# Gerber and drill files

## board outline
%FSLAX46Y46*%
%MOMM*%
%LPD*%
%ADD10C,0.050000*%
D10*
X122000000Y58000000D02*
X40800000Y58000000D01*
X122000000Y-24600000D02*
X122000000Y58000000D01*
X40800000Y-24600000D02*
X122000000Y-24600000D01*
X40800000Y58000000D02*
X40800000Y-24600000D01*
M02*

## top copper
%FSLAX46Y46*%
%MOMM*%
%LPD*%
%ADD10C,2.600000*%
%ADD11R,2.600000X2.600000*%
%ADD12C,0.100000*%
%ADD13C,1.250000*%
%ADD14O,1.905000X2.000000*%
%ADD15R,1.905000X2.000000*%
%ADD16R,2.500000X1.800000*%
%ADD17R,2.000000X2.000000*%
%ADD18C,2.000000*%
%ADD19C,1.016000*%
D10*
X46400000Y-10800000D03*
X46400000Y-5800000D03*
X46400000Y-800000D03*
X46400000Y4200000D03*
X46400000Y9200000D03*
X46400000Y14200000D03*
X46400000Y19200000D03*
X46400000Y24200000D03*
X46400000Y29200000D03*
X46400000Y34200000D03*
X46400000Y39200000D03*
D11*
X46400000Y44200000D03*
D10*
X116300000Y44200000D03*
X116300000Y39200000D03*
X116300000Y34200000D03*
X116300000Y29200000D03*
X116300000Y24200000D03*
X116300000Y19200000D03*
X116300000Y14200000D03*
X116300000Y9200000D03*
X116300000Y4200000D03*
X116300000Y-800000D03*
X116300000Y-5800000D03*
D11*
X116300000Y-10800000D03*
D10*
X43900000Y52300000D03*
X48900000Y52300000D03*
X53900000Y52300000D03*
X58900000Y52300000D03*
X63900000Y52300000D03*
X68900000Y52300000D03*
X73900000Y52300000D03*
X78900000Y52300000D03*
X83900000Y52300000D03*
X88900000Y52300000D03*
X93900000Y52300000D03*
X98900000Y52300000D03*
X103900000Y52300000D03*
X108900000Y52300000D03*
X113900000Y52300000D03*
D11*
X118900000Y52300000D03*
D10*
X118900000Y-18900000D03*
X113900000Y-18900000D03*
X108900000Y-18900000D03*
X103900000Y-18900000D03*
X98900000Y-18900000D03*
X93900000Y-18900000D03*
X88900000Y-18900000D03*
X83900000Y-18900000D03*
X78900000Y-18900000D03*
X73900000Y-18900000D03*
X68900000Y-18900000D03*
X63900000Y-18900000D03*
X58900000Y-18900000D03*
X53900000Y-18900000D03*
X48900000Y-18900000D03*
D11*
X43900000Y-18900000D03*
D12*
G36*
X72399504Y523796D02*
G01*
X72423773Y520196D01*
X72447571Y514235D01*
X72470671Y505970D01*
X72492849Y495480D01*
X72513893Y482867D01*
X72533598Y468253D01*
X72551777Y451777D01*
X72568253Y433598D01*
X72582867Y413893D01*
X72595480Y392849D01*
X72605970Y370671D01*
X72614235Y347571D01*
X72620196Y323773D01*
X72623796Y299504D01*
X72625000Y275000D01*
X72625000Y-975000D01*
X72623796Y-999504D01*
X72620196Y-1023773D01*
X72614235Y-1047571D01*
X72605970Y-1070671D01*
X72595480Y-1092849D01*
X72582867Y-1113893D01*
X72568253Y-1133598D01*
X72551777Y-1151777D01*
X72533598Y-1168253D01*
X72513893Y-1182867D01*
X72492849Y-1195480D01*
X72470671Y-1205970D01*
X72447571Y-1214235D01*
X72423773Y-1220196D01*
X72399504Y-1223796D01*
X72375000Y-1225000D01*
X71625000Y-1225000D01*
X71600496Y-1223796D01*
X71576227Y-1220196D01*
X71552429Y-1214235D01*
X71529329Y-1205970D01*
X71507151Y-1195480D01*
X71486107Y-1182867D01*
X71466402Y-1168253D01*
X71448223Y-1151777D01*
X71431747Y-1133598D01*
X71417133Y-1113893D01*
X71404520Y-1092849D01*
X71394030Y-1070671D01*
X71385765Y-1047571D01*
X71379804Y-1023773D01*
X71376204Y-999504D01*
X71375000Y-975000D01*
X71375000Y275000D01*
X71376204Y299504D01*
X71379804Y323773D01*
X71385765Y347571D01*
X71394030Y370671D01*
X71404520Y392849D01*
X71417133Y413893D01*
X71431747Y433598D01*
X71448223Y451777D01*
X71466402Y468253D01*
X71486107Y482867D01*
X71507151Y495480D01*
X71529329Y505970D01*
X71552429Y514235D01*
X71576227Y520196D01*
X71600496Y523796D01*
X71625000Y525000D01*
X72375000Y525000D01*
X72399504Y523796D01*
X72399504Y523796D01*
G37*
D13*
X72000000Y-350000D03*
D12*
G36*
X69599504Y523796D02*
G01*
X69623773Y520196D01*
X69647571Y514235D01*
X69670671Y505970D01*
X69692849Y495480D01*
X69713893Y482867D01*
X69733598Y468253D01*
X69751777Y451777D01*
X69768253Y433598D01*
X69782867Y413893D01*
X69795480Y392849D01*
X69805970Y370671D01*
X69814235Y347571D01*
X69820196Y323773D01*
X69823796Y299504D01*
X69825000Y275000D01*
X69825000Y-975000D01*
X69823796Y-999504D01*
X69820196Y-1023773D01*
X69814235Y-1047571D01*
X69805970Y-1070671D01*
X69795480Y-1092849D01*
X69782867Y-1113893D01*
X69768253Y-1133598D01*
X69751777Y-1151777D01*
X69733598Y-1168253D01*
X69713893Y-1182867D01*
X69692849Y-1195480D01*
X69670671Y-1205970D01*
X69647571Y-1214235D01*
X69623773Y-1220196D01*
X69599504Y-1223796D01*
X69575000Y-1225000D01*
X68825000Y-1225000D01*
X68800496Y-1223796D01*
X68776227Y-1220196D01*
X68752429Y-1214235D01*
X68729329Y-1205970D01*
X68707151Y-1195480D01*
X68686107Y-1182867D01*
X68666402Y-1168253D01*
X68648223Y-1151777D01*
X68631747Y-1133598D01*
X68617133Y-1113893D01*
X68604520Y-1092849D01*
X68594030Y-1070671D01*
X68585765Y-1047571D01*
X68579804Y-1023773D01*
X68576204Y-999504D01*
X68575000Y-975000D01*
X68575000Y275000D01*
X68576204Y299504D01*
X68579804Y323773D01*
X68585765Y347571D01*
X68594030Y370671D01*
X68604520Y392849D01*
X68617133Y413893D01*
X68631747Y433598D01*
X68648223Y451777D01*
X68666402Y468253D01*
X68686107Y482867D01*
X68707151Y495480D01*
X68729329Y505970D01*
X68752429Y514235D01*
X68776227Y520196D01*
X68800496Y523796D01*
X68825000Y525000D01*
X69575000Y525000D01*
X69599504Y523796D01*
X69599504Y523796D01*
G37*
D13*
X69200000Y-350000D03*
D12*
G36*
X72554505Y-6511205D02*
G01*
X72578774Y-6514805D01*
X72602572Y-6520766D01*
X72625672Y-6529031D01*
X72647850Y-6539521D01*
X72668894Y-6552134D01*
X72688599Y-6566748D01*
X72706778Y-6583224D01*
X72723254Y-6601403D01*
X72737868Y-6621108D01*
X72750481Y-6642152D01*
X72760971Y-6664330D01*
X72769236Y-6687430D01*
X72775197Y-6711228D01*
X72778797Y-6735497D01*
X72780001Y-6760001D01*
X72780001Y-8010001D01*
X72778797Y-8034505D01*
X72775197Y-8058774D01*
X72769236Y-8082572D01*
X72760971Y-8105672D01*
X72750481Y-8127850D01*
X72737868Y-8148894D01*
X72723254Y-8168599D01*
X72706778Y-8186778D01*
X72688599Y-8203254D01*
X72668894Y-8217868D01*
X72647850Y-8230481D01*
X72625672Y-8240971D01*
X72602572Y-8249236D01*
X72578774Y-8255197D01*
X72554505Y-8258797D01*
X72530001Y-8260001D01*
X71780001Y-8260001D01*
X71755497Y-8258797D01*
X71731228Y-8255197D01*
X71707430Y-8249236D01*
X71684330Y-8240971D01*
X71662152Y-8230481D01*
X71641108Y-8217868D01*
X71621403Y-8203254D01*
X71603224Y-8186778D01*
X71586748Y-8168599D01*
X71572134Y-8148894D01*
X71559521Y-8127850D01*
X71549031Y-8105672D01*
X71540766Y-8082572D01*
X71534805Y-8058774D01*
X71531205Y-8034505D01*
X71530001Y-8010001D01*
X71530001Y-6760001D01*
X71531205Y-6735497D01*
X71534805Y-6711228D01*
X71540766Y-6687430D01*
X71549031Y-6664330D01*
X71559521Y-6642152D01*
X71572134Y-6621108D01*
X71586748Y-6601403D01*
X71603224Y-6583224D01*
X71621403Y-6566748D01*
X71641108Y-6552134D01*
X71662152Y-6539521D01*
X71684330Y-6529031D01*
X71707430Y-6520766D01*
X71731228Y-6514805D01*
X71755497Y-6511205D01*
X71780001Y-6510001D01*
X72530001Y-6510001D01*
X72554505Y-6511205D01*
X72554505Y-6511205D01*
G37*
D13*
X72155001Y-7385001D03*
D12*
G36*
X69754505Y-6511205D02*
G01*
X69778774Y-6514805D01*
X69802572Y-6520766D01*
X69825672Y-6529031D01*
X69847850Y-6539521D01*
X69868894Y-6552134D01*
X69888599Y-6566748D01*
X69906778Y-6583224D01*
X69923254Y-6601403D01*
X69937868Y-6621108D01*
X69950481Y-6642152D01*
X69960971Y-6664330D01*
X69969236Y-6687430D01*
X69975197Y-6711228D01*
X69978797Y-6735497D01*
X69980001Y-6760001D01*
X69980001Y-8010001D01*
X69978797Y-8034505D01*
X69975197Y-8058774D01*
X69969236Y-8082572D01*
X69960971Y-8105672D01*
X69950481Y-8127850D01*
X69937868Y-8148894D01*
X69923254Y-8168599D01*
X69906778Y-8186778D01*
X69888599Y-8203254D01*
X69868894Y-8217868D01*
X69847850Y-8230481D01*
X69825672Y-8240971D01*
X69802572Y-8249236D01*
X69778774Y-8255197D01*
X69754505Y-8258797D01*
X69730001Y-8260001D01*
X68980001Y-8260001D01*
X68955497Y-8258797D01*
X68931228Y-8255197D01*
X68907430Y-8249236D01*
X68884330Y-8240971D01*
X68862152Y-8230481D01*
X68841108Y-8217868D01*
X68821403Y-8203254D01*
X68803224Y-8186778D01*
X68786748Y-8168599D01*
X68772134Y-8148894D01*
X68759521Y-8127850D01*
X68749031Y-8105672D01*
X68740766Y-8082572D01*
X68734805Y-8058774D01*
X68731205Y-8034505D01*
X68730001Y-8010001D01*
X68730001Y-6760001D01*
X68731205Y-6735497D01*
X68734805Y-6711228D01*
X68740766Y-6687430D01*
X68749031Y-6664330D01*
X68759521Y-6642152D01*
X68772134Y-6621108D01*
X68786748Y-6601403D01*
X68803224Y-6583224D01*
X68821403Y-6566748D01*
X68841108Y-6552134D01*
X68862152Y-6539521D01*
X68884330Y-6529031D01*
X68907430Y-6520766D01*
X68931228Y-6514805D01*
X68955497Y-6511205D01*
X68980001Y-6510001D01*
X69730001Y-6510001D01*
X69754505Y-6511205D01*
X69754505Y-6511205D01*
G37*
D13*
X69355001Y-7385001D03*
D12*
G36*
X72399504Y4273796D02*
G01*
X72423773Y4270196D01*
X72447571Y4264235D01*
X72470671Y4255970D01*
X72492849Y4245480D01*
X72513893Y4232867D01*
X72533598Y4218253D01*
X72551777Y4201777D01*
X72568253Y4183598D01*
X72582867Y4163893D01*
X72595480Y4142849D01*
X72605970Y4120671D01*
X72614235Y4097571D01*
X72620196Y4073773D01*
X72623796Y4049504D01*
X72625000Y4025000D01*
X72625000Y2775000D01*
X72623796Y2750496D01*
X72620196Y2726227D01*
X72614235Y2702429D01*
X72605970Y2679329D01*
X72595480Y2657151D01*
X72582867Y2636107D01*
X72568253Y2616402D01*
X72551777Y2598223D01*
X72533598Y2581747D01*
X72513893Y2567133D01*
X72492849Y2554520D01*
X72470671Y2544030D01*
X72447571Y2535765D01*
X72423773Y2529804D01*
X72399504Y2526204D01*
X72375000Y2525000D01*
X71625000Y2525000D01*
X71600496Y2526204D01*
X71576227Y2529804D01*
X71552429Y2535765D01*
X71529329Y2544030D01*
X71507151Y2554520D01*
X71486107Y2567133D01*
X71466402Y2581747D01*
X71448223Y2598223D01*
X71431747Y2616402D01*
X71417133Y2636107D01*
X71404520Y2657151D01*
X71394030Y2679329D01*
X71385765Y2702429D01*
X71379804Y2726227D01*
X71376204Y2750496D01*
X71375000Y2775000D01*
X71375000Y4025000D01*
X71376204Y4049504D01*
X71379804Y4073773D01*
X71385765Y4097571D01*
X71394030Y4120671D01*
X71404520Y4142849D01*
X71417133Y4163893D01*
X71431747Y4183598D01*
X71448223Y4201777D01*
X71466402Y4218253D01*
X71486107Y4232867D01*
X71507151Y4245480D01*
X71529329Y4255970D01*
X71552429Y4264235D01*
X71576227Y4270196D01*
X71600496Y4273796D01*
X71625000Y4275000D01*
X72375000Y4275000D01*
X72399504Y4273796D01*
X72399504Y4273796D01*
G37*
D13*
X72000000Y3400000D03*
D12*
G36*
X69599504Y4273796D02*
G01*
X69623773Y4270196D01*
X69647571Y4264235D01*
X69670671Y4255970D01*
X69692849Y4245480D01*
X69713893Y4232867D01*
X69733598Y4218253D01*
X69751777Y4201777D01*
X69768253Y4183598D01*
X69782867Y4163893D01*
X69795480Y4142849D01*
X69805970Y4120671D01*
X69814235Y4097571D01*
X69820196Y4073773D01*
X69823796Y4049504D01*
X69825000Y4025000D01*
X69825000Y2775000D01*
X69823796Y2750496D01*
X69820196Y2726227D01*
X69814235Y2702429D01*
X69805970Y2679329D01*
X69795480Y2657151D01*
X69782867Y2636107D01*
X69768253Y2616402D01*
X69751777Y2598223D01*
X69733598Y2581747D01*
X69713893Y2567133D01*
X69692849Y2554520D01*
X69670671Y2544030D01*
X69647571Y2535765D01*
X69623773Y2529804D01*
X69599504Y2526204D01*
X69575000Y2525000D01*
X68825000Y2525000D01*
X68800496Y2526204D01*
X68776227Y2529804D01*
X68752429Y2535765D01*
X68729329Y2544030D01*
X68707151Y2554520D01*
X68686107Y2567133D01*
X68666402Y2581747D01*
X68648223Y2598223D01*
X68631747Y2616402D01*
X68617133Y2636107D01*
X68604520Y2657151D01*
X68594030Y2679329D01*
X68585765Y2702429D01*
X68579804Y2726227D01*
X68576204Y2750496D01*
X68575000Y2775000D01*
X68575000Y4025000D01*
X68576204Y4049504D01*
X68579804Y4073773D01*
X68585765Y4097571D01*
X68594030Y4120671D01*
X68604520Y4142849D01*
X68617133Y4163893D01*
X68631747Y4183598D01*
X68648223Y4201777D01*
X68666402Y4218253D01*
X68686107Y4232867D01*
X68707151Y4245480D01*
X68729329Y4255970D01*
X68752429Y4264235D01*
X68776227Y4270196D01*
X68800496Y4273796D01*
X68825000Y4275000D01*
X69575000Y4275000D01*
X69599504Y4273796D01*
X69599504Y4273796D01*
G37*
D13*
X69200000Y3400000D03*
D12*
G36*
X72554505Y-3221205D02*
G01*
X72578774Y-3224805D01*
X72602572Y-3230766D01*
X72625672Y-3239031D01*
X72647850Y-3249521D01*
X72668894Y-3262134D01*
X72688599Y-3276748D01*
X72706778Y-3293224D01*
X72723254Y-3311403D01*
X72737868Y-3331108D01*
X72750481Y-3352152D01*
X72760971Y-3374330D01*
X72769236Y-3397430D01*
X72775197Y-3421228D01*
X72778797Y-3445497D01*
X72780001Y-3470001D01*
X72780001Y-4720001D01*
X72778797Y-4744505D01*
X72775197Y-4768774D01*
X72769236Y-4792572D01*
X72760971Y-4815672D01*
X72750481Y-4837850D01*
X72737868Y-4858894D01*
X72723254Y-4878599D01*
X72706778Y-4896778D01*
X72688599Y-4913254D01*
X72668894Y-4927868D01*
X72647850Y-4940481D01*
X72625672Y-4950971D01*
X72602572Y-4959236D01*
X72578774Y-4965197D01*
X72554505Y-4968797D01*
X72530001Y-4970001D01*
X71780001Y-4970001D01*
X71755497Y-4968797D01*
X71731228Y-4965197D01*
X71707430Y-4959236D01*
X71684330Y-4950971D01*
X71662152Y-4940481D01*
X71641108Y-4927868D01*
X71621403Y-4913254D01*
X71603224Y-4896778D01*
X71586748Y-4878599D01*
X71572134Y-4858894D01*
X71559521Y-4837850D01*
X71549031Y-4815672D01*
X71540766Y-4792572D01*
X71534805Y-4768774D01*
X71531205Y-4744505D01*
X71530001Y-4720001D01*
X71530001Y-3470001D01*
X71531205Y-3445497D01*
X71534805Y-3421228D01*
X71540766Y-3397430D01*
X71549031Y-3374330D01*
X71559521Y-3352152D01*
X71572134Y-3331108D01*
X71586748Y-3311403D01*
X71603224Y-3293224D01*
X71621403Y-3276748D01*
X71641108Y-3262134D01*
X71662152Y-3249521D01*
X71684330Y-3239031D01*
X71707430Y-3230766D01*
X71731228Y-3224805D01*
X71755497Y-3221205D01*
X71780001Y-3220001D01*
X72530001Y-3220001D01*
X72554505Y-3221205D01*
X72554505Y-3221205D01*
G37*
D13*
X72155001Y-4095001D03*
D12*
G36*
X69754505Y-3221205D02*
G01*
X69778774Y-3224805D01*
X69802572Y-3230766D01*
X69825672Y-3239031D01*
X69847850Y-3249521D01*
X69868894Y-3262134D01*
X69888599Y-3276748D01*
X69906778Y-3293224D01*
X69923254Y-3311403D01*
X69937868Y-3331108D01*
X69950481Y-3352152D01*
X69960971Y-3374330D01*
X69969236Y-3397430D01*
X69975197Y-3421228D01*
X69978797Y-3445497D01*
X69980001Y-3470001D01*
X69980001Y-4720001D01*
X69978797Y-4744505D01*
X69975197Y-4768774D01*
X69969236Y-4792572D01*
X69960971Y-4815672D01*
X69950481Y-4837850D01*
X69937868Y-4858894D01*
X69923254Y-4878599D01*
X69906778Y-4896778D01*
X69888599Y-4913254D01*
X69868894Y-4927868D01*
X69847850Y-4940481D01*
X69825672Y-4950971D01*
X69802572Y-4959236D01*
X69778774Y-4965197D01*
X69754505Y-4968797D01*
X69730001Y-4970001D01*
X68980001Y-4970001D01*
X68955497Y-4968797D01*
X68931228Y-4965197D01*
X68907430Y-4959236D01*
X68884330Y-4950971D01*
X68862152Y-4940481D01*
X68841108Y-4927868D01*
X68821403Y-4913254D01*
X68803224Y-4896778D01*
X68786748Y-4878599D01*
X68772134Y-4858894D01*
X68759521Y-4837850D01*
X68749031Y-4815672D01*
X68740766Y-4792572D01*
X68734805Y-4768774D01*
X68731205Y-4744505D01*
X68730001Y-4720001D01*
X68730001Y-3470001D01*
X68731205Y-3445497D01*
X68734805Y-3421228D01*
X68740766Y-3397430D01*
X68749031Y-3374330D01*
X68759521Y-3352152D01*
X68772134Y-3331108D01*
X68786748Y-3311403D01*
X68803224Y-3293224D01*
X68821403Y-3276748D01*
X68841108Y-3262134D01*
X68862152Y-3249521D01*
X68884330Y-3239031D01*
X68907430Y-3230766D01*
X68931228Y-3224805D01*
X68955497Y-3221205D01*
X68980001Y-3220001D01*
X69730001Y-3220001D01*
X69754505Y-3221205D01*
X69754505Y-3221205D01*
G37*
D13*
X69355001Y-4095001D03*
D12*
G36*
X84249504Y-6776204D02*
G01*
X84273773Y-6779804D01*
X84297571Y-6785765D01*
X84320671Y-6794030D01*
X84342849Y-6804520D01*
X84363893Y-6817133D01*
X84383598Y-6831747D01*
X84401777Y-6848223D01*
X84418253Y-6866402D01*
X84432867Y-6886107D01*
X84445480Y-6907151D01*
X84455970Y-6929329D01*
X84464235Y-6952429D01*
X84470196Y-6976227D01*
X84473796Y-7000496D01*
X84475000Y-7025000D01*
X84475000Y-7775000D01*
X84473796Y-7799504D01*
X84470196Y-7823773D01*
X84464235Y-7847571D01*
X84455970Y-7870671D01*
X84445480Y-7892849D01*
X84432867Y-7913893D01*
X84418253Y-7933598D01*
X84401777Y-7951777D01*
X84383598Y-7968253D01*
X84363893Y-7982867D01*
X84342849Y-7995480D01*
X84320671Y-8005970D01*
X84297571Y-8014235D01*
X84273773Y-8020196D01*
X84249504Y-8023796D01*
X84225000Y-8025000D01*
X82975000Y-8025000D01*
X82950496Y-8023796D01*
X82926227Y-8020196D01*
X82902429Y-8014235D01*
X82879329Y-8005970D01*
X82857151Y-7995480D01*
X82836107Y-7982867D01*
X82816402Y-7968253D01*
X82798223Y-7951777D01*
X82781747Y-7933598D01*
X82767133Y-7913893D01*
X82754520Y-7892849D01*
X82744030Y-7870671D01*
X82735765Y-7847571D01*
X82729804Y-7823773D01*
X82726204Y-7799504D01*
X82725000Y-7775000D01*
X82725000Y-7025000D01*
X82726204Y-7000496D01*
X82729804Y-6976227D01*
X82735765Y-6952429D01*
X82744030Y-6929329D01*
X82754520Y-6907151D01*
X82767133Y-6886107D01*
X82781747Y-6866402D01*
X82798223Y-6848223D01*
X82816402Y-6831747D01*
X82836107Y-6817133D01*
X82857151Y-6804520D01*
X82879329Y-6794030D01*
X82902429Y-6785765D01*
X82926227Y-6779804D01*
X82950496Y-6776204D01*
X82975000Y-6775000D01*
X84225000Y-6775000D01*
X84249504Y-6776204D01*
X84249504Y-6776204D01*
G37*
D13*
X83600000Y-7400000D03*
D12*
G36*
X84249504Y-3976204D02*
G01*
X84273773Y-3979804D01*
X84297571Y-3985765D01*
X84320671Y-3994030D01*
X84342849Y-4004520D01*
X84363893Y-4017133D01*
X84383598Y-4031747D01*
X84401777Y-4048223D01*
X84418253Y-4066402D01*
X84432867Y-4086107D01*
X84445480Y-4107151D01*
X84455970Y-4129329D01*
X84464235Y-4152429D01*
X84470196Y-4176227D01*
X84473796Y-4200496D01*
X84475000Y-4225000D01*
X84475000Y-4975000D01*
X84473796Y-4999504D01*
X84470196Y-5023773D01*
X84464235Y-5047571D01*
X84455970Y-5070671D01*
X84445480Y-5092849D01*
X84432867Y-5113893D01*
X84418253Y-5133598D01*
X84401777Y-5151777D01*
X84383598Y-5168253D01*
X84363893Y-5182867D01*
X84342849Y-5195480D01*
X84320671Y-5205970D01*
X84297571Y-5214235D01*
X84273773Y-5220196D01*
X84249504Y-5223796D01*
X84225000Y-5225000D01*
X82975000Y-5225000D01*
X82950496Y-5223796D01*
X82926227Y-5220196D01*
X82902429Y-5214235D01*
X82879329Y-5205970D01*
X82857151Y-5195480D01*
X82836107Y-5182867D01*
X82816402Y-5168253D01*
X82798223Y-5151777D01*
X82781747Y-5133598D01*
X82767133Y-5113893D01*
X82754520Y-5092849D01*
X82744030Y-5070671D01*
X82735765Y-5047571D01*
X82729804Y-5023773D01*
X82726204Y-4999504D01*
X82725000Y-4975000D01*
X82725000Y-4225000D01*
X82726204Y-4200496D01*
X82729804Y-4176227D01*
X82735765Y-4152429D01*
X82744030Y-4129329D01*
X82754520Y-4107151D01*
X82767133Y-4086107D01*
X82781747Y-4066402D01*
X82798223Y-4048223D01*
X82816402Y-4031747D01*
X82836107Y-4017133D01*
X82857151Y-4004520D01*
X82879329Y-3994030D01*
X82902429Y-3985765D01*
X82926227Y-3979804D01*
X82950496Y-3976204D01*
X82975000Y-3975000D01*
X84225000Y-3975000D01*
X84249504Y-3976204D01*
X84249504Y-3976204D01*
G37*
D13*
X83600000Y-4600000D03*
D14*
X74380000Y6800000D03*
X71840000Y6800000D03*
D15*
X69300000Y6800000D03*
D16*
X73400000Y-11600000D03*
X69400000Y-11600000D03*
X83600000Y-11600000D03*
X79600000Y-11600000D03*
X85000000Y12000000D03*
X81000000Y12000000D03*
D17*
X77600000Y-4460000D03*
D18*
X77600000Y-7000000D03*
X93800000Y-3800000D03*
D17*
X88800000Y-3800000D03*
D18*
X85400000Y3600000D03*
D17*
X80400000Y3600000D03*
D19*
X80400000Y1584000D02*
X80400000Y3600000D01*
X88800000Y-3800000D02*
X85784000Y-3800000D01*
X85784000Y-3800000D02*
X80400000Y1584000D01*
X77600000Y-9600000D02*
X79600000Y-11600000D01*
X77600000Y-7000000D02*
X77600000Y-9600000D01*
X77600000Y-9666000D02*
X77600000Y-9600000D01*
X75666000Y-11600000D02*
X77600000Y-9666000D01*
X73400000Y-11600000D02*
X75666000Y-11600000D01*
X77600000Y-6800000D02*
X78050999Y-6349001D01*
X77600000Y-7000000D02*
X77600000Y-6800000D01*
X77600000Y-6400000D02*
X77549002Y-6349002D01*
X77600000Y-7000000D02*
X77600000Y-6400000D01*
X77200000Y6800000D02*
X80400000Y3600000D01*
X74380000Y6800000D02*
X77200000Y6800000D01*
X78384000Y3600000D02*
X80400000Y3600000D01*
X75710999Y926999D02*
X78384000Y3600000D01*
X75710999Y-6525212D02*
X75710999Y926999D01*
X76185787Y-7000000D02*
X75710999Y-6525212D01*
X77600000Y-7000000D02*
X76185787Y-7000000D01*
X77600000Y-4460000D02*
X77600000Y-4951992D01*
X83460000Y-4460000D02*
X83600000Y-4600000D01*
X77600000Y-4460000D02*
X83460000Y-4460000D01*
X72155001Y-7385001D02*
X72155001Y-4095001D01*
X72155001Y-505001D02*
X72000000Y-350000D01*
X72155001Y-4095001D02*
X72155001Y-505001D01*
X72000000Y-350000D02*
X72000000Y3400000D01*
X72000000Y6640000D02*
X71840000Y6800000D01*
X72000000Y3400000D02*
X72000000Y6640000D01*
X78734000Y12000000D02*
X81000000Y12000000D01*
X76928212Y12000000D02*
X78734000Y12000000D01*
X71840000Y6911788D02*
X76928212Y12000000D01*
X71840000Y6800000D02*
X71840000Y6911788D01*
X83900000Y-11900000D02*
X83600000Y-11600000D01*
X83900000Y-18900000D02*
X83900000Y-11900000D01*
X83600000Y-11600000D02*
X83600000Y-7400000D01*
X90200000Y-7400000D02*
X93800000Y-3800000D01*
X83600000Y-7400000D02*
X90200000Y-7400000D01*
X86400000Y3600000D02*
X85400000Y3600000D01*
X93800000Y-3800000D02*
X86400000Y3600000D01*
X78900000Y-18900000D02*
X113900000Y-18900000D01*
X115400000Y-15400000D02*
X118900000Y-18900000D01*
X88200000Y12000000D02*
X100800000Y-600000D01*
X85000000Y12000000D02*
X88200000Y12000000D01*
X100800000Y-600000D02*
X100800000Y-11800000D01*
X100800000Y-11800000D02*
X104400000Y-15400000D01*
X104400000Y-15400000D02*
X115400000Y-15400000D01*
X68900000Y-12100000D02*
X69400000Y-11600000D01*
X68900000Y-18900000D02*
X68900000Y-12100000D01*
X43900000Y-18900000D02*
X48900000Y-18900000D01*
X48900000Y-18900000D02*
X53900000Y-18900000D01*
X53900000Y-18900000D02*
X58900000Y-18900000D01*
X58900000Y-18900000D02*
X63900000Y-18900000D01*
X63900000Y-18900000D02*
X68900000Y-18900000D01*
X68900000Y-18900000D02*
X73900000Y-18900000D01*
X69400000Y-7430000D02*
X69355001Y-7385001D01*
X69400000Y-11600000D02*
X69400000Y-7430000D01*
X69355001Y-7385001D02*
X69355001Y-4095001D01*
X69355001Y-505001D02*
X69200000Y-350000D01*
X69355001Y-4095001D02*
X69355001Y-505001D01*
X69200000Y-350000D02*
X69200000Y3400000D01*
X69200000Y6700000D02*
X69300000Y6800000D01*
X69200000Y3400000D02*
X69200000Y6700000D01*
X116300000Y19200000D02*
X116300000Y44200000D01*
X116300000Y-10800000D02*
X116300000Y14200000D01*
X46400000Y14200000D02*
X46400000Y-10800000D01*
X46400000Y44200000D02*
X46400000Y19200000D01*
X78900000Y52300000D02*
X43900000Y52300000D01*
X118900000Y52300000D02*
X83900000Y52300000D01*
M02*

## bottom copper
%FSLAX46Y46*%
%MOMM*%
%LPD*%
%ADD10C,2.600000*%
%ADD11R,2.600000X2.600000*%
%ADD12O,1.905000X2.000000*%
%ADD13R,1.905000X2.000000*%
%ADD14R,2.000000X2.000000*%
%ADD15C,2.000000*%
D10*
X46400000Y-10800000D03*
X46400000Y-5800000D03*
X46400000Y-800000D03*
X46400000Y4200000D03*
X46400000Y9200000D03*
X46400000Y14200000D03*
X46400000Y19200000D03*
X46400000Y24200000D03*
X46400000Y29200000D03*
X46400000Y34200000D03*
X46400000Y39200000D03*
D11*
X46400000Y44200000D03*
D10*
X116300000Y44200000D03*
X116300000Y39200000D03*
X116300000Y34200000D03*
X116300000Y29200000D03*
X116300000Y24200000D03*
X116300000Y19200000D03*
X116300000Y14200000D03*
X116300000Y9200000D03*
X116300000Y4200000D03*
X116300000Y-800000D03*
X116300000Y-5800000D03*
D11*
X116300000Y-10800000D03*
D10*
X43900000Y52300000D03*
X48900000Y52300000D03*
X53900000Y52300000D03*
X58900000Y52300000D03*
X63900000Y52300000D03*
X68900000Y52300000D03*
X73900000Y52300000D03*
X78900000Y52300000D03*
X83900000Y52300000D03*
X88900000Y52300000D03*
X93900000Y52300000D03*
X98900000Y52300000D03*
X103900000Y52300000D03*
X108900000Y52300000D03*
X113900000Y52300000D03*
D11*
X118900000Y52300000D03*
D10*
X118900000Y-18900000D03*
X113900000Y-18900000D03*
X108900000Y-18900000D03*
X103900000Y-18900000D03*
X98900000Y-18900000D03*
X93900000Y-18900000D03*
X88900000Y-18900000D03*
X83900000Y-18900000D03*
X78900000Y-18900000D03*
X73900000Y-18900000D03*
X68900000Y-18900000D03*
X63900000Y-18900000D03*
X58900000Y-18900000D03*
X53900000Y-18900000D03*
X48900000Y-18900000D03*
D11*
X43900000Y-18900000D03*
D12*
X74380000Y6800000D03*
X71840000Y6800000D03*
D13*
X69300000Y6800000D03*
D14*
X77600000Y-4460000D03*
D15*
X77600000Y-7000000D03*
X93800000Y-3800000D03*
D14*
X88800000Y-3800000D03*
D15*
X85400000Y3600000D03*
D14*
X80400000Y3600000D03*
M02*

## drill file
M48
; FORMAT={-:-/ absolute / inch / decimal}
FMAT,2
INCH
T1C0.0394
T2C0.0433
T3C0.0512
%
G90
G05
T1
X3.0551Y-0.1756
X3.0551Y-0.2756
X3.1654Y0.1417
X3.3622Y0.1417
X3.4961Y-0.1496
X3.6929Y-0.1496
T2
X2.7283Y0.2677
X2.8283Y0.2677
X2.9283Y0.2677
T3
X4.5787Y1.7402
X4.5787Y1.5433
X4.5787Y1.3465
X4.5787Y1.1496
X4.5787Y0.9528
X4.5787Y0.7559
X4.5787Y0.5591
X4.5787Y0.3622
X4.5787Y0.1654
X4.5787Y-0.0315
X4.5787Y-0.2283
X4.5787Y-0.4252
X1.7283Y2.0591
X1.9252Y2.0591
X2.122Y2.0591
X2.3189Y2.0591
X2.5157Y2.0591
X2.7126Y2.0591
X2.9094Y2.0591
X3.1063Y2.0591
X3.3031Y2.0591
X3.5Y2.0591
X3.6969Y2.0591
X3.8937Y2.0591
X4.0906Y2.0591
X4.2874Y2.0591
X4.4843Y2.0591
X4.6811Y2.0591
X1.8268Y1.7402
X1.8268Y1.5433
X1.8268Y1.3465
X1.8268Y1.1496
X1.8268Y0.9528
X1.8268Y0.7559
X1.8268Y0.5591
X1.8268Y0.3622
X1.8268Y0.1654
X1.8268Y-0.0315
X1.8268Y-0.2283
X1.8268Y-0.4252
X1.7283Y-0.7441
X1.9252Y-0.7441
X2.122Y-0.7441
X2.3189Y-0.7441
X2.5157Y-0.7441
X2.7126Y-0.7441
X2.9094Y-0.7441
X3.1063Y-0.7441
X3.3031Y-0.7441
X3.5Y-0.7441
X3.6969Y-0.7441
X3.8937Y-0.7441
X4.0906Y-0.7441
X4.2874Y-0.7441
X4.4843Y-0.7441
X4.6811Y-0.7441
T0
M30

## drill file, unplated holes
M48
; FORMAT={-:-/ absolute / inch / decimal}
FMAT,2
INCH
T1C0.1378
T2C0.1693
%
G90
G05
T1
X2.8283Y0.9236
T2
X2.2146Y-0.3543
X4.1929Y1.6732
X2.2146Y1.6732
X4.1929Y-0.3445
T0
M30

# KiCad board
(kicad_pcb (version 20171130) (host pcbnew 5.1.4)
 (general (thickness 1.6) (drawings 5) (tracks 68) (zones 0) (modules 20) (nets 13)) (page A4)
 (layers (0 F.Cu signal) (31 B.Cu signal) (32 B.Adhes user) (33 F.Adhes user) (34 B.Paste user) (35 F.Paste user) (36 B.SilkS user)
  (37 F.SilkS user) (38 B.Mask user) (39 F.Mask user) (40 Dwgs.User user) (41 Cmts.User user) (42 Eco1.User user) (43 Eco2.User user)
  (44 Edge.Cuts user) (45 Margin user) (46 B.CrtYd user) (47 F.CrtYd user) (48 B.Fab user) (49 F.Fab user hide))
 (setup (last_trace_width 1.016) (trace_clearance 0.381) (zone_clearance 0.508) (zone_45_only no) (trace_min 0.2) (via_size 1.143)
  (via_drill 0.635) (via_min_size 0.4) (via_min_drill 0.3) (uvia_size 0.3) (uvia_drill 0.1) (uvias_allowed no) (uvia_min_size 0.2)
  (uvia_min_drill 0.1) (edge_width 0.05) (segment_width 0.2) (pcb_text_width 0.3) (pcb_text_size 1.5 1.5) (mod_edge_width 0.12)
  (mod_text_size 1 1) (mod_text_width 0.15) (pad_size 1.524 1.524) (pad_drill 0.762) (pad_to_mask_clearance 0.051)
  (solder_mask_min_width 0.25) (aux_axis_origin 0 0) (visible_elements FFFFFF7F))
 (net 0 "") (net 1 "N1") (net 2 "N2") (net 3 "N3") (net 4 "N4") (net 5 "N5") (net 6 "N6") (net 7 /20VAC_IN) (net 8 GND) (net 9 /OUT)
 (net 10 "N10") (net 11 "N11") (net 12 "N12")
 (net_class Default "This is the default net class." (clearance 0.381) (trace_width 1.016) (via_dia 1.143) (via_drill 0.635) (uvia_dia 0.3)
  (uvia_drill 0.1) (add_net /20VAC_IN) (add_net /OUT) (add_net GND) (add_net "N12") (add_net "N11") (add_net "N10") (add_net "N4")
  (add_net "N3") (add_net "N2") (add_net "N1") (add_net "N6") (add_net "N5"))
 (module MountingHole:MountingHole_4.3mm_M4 (layer F.Cu) (at 56.25 -42.5)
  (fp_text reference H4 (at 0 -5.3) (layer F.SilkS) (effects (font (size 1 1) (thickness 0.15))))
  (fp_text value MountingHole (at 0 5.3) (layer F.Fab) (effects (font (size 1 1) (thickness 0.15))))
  (pad 1 np_thru_hole circle (at 0 0) (size 4.3 4.3) (drill 4.3) (layers *.Cu *.Mask)))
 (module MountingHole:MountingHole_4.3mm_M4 (layer F.Cu) (at 106.5 -42.5)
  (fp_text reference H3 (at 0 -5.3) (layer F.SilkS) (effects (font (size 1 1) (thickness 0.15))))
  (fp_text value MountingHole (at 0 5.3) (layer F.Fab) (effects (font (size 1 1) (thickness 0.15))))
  (pad 1 np_thru_hole circle (at 0 0) (size 4.3 4.3) (drill 4.3) (layers *.Cu *.Mask)))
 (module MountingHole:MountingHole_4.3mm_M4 (layer F.Cu) (at 56.25 9)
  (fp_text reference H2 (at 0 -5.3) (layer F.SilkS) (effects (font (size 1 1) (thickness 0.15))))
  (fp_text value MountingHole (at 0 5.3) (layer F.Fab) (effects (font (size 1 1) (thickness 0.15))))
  (pad 1 np_thru_hole circle (at 0 0) (size 4.3 4.3) (drill 4.3) (layers *.Cu *.Mask)))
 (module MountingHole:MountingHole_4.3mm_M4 (layer F.Cu) (at 106.5 8.75)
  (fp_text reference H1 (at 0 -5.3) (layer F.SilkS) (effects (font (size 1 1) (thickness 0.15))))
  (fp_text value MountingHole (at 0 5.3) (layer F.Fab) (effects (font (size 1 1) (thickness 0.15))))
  (pad 1 np_thru_hole circle (at 0 0) (size 4.3 4.3) (drill 4.3) (layers *.Cu *.Mask)))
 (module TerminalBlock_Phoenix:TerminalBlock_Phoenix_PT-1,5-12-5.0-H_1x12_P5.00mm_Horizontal (layer F.Cu) (at 46.4 -44.2 270)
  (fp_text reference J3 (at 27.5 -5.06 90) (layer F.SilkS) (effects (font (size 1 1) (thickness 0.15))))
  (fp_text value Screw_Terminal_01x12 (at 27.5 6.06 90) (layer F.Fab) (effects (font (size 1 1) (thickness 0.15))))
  (pad 12 thru_hole circle (at 55 0 270) (size 2.6 2.6) (drill 1.3) (layers *.Cu *.Mask) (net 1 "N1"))
  (pad 11 thru_hole circle (at 50 0 270) (size 2.6 2.6) (drill 1.3) (layers *.Cu *.Mask) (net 1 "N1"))
  (pad 10 thru_hole circle (at 45 0 270) (size 2.6 2.6) (drill 1.3) (layers *.Cu *.Mask) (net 1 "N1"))
  (pad 9 thru_hole circle (at 40 0 270) (size 2.6 2.6) (drill 1.3) (layers *.Cu *.Mask) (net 1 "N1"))
  (pad 8 thru_hole circle (at 35 0 270) (size 2.6 2.6) (drill 1.3) (layers *.Cu *.Mask) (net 1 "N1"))
  (pad 7 thru_hole circle (at 30 0 270) (size 2.6 2.6) (drill 1.3) (layers *.Cu *.Mask) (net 1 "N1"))
  (pad 6 thru_hole circle (at 25 0 270) (size 2.6 2.6) (drill 1.3) (layers *.Cu *.Mask) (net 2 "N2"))
  (pad 5 thru_hole circle (at 20 0 270) (size 2.6 2.6) (drill 1.3) (layers *.Cu *.Mask) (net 2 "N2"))
  (pad 4 thru_hole circle (at 15 0 270) (size 2.6 2.6) (drill 1.3) (layers *.Cu *.Mask) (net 2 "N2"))
  (pad 3 thru_hole circle (at 10 0 270) (size 2.6 2.6) (drill 1.3) (layers *.Cu *.Mask) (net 2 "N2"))
  (pad 2 thru_hole circle (at 5 0 270) (size 2.6 2.6) (drill 1.3) (layers *.Cu *.Mask) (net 2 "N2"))
  (pad 1 thru_hole rect (at 0 0 270) (size 2.6 2.6) (drill 1.3) (layers *.Cu *.Mask) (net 2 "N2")))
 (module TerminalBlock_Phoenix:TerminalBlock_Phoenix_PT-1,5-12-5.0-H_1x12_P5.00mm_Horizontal (layer F.Cu) (at 116.3 10.8 90)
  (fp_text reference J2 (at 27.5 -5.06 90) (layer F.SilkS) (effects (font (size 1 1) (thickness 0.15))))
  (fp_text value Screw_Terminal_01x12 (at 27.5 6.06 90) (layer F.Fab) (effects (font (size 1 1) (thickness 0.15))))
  (pad 12 thru_hole circle (at 55 0 90) (size 2.6 2.6) (drill 1.3) (layers *.Cu *.Mask) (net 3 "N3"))
  (pad 11 thru_hole circle (at 50 0 90) (size 2.6 2.6) (drill 1.3) (layers *.Cu *.Mask) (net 3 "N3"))
  (pad 10 thru_hole circle (at 45 0 90) (size 2.6 2.6) (drill 1.3) (layers *.Cu *.Mask) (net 3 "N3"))
  (pad 9 thru_hole circle (at 40 0 90) (size 2.6 2.6) (drill 1.3) (layers *.Cu *.Mask) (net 3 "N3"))
  (pad 8 thru_hole circle (at 35 0 90) (size 2.6 2.6) (drill 1.3) (layers *.Cu *.Mask) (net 3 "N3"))
  (pad 7 thru_hole circle (at 30 0 90) (size 2.6 2.6) (drill 1.3) (layers *.Cu *.Mask) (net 3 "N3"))
  (pad 6 thru_hole circle (at 25 0 90) (size 2.6 2.6) (drill 1.3) (layers *.Cu *.Mask) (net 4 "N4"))
  (pad 5 thru_hole circle (at 20 0 90) (size 2.6 2.6) (drill 1.3) (layers *.Cu *.Mask) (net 4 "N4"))
  (pad 4 thru_hole circle (at 15 0 90) (size 2.6 2.6) (drill 1.3) (layers *.Cu *.Mask) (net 4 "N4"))
  (pad 3 thru_hole circle (at 10 0 90) (size 2.6 2.6) (drill 1.3) (layers *.Cu *.Mask) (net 4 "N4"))
  (pad 2 thru_hole circle (at 5 0 90) (size 2.6 2.6) (drill 1.3) (layers *.Cu *.Mask) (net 4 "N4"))
  (pad 1 thru_hole rect (at 0 0 90) (size 2.6 2.6) (drill 1.3) (layers *.Cu *.Mask) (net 4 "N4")))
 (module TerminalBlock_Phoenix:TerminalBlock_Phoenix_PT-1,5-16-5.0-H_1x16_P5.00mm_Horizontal (layer F.Cu) (at 118.9 -52.3 180)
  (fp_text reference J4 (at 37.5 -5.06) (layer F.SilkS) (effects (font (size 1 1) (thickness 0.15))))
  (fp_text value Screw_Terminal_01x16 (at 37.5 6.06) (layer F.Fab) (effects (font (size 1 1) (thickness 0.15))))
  (pad 16 thru_hole circle (at 75 0 180) (size 2.6 2.6) (drill 1.3) (layers *.Cu *.Mask) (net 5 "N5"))
  (pad 15 thru_hole circle (at 70 0 180) (size 2.6 2.6) (drill 1.3) (layers *.Cu *.Mask) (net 5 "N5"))
  (pad 14 thru_hole circle (at 65 0 180) (size 2.6 2.6) (drill 1.3) (layers *.Cu *.Mask) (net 5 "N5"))
  (pad 13 thru_hole circle (at 60 0 180) (size 2.6 2.6) (drill 1.3) (layers *.Cu *.Mask) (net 5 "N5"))
  (pad 12 thru_hole circle (at 55 0 180) (size 2.6 2.6) (drill 1.3) (layers *.Cu *.Mask) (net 5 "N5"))
  (pad 11 thru_hole circle (at 50 0 180) (size 2.6 2.6) (drill 1.3) (layers *.Cu *.Mask) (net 5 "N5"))
  (pad 10 thru_hole circle (at 45 0 180) (size 2.6 2.6) (drill 1.3) (layers *.Cu *.Mask) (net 5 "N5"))
  (pad 9 thru_hole circle (at 40 0 180) (size 2.6 2.6) (drill 1.3) (layers *.Cu *.Mask) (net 5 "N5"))
  (pad 8 thru_hole circle (at 35 0 180) (size 2.6 2.6) (drill 1.3) (layers *.Cu *.Mask) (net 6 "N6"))
  (pad 7 thru_hole circle (at 30 0 180) (size 2.6 2.6) (drill 1.3) (layers *.Cu *.Mask) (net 6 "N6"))
  (pad 6 thru_hole circle (at 25 0 180) (size 2.6 2.6) (drill 1.3) (layers *.Cu *.Mask) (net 6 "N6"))
  (pad 5 thru_hole circle (at 20 0 180) (size 2.6 2.6) (drill 1.3) (layers *.Cu *.Mask) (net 6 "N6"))
  (pad 4 thru_hole circle (at 15 0 180) (size 2.6 2.6) (drill 1.3) (layers *.Cu *.Mask) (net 6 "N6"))
  (pad 3 thru_hole circle (at 10 0 180) (size 2.6 2.6) (drill 1.3) (layers *.Cu *.Mask) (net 6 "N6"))
  (pad 2 thru_hole circle (at 5 0 180) (size 2.6 2.6) (drill 1.3) (layers *.Cu *.Mask) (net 6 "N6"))
  (pad 1 thru_hole rect (at 0 0 180) (size 2.6 2.6) (drill 1.3) (layers *.Cu *.Mask) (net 6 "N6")))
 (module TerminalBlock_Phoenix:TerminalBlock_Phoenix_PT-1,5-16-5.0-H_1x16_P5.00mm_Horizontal (layer F.Cu) (at 43.9 18.9)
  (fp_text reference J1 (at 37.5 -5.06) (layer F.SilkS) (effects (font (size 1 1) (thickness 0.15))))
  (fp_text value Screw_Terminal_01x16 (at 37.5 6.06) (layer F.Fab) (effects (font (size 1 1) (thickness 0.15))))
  (pad 16 thru_hole circle (at 75 0) (size 2.6 2.6) (drill 1.3) (layers *.Cu *.Mask) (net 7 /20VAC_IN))
  (pad 15 thru_hole circle (at 70 0) (size 2.6 2.6) (drill 1.3) (layers *.Cu *.Mask) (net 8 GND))
  (pad 14 thru_hole circle (at 65 0) (size 2.6 2.6) (drill 1.3) (layers *.Cu *.Mask) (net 8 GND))
  (pad 13 thru_hole circle (at 60 0) (size 2.6 2.6) (drill 1.3) (layers *.Cu *.Mask) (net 8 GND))
  (pad 12 thru_hole circle (at 55 0) (size 2.6 2.6) (drill 1.3) (layers *.Cu *.Mask) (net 8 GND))
  (pad 11 thru_hole circle (at 50 0) (size 2.6 2.6) (drill 1.3) (layers *.Cu *.Mask) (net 8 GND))
  (pad 10 thru_hole circle (at 45 0) (size 2.6 2.6) (drill 1.3) (layers *.Cu *.Mask) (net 8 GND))
  (pad 9 thru_hole circle (at 40 0) (size 2.6 2.6) (drill 1.3) (layers *.Cu *.Mask) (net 8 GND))
  (pad 8 thru_hole circle (at 35 0) (size 2.6 2.6) (drill 1.3) (layers *.Cu *.Mask) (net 8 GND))
  (pad 7 thru_hole circle (at 30 0) (size 2.6 2.6) (drill 1.3) (layers *.Cu *.Mask) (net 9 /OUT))
  (pad 6 thru_hole circle (at 25 0) (size 2.6 2.6) (drill 1.3) (layers *.Cu *.Mask) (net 9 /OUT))
  (pad 5 thru_hole circle (at 20 0) (size 2.6 2.6) (drill 1.3) (layers *.Cu *.Mask) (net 9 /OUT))
  (pad 4 thru_hole circle (at 15 0) (size 2.6 2.6) (drill 1.3) (layers *.Cu *.Mask) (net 9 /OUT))
  (pad 3 thru_hole circle (at 10 0) (size 2.6 2.6) (drill 1.3) (layers *.Cu *.Mask) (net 9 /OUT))
  (pad 2 thru_hole circle (at 5 0) (size 2.6 2.6) (drill 1.3) (layers *.Cu *.Mask) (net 9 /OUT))
  (pad 1 thru_hole rect (at 0 0) (size 2.6 2.6) (drill 1.3) (layers *.Cu *.Mask) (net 9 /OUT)))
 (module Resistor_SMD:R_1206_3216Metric (layer F.Cu) (at 70.6 0.35)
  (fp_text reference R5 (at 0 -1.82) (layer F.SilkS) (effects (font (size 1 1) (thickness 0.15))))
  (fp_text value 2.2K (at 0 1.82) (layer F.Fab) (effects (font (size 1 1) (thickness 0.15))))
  (pad 2 smd roundrect (at 1.4 0) (size 1.25 1.75) (layers F.Cu F.Paste F.Mask) (roundrect_rratio 0.2) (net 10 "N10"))
  (pad 1 smd roundrect (at -1.4 0) (size 1.25 1.75) (layers F.Cu F.Paste F.Mask) (roundrect_rratio 0.2) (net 9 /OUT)))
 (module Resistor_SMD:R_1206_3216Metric (layer F.Cu) (at 70.755001 7.385001)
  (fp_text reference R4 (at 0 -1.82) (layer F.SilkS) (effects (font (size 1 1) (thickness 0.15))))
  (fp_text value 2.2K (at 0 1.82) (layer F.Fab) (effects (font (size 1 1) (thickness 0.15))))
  (pad 2 smd roundrect (at 1.4 0) (size 1.25 1.75) (layers F.Cu F.Paste F.Mask) (roundrect_rratio 0.2) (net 10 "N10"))
  (pad 1 smd roundrect (at -1.4 0) (size 1.25 1.75) (layers F.Cu F.Paste F.Mask) (roundrect_rratio 0.2) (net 9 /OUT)))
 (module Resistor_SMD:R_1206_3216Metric (layer F.Cu) (at 70.6 -3.4)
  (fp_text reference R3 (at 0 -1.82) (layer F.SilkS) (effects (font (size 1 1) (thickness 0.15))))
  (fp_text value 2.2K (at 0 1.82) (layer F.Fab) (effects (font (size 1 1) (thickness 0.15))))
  (pad 2 smd roundrect (at 1.4 0) (size 1.25 1.75) (layers F.Cu F.Paste F.Mask) (roundrect_rratio 0.2) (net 10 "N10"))
  (pad 1 smd roundrect (at -1.4 0) (size 1.25 1.75) (layers F.Cu F.Paste F.Mask) (roundrect_rratio 0.2) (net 9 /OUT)))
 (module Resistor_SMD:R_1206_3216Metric (layer F.Cu) (at 70.755001 4.095001)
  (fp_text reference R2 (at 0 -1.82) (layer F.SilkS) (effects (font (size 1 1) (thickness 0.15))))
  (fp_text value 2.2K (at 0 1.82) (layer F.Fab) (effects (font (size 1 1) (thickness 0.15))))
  (pad 2 smd roundrect (at 1.4 0) (size 1.25 1.75) (layers F.Cu F.Paste F.Mask) (roundrect_rratio 0.2) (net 10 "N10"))
  (pad 1 smd roundrect (at -1.4 0) (size 1.25 1.75) (layers F.Cu F.Paste F.Mask) (roundrect_rratio 0.2) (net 9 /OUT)))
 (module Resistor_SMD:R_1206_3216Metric (layer F.Cu) (at 83.6 6 270)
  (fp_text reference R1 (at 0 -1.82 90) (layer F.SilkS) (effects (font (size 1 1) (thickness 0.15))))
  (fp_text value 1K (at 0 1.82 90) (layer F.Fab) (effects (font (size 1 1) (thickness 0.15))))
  (pad 2 smd roundrect (at 1.4 0 270) (size 1.25 1.75) (layers F.Cu F.Paste F.Mask) (roundrect_rratio 0.2) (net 8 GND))
  (pad 1 smd roundrect (at -1.4 0 270) (size 1.25 1.75) (layers F.Cu F.Paste F.Mask) (roundrect_rratio 0.2) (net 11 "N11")))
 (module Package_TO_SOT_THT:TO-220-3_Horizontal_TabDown (layer F.Cu) (at 69.3 -6.8)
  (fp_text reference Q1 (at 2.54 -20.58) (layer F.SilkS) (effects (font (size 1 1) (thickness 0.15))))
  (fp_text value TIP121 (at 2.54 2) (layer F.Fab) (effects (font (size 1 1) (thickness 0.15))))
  (pad 3 thru_hole oval (at 5.08 0) (size 1.905 2) (drill 1.1) (layers *.Cu *.Mask) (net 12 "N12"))
  (pad 2 thru_hole oval (at 2.54 0) (size 1.905 2) (drill 1.1) (layers *.Cu *.Mask) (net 10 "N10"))
  (pad 1 thru_hole rect (at 0 0) (size 1.905 2) (drill 1.1) (layers *.Cu *.Mask) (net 9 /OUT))
  (pad "" np_thru_hole oval (at 2.54 -16.66) (size 3.5 3.5) (drill 3.5) (layers *.Cu *.Mask)))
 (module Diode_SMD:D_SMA (layer F.Cu) (at 71.4 11.6)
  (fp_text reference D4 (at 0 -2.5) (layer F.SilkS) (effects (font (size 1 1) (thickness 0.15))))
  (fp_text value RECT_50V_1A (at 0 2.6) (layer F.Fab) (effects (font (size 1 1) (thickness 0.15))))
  (pad 2 smd rect (at 2 0) (size 2.5 1.8) (layers F.Cu F.Paste F.Mask) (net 12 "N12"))
  (pad 1 smd rect (at -2 0) (size 2.5 1.8) (layers F.Cu F.Paste F.Mask) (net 9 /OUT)))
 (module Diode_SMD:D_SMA (layer F.Cu) (at 81.6 11.6)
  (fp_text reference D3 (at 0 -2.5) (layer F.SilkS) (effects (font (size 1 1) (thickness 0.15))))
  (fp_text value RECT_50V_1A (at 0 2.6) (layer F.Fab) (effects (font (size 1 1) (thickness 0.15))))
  (pad 2 smd rect (at 2 0) (size 2.5 1.8) (layers F.Cu F.Paste F.Mask) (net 8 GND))
  (pad 1 smd rect (at -2 0) (size 2.5 1.8) (layers F.Cu F.Paste F.Mask) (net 12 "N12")))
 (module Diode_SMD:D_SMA (layer F.Cu) (at 83 -12)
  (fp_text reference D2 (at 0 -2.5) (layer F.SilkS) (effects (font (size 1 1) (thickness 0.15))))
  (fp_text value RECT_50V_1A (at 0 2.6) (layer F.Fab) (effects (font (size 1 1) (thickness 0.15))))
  (pad 2 smd rect (at 2 0) (size 2.5 1.8) (layers F.Cu F.Paste F.Mask) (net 7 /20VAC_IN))
  (pad 1 smd rect (at -2 0) (size 2.5 1.8) (layers F.Cu F.Paste F.Mask) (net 10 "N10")))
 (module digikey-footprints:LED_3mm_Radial (layer F.Cu) (at 77.6 7 270)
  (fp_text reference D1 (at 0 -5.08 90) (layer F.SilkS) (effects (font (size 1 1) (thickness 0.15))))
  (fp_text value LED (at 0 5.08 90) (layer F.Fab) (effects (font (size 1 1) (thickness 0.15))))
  (pad 1 thru_hole rect (at -2.54 0 270) (size 2 2) (drill 1) (layers *.Cu *.Mask) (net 11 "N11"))
  (pad 2 thru_hole circle (at 0 0 270) (size 2 2) (drill 1) (layers *.Cu *.Mask) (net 12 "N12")))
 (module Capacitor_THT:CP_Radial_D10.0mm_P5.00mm (layer F.Cu) (at 88.8 3.8)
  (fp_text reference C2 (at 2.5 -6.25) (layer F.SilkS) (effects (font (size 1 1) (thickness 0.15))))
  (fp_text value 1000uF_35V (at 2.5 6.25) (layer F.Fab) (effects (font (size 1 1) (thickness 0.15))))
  (pad 2 thru_hole circle (at 5 0) (size 2 2) (drill 1) (layers *.Cu *.Mask) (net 8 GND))
  (pad 1 thru_hole rect (at 0 0) (size 2 2) (drill 1) (layers *.Cu *.Mask) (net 12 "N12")))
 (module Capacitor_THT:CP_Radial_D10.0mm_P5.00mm (layer F.Cu) (at 80.4 -3.6)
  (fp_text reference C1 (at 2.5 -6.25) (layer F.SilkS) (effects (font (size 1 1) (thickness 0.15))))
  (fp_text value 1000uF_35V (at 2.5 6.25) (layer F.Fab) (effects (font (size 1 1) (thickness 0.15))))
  (pad 2 thru_hole circle (at 5 0) (size 2 2) (drill 1) (layers *.Cu *.Mask) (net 8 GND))
  (pad 1 thru_hole rect (at 0 0) (size 2 2) (drill 1) (layers *.Cu *.Mask) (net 12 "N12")))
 (gr_line (start 122 -58) (end 40.8 -58) (layer Edge.Cuts) (width 0.05))
 (gr_line (start 122 24.6) (end 122 -58) (layer Edge.Cuts) (width 0.05))
 (gr_line (start 40.8 24.6) (end 122 24.6) (layer Edge.Cuts) (width 0.05))
 (gr_line (start 40.8 -58) (end 40.8 24.6) (layer Edge.Cuts) (width 0.05))
 (segment (start 80.4 -1.584) (end 80.4 -3.6) (width 1.016) (layer F.Cu) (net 12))
 (segment (start 88.8 3.8) (end 85.784 3.8) (width 1.016) (layer F.Cu) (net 12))
 (segment (start 85.784 3.8) (end 80.4 -1.584) (width 1.016) (layer F.Cu) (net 12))
 (segment (start 77.6 9.6) (end 79.6 11.6) (width 1.016) (layer F.Cu) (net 12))
 (segment (start 77.6 7) (end 77.6 9.6) (width 1.016) (layer F.Cu) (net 12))
 (segment (start 77.6 9.666) (end 77.6 9.6) (width 1.016) (layer F.Cu) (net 12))
 (segment (start 75.666 11.6) (end 77.6 9.666) (width 1.016) (layer F.Cu) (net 12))
 (segment (start 73.4 11.6) (end 75.666 11.6) (width 1.016) (layer F.Cu) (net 12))
 (segment (start 77.6 6.8) (end 78.050999 6.349001) (width 1.016) (layer F.Cu) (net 12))
 (segment (start 77.6 7) (end 77.6 6.8) (width 1.016) (layer F.Cu) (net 12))
 (segment (start 77.6 6.4) (end 77.549002 6.349002) (width 1.016) (layer F.Cu) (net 12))
 (segment (start 77.6 7) (end 77.6 6.4) (width 1.016) (layer F.Cu) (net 12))
 (segment (start 77.2 -6.8) (end 80.4 -3.6) (width 1.016) (layer F.Cu) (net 12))
 (segment (start 74.38 -6.8) (end 77.2 -6.8) (width 1.016) (layer F.Cu) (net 12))
 (segment (start 78.384 -3.6) (end 80.4 -3.6) (width 1.016) (layer F.Cu) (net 12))
 (segment (start 75.710999 -0.926999) (end 78.384 -3.6) (width 1.016) (layer F.Cu) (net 12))
 (segment (start 75.710999 6.525212) (end 75.710999 -0.926999) (width 1.016) (layer F.Cu) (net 12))
 (segment (start 76.185787 7) (end 75.710999 6.525212) (width 1.016) (layer F.Cu) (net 12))
 (segment (start 77.6 7) (end 76.185787 7) (width 1.016) (layer F.Cu) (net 12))
 (segment (start 77.6 4.46) (end 77.6 4.951992) (width 1.016) (layer F.Cu) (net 11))
 (segment (start 83.46 4.46) (end 83.6 4.6) (width 1.016) (layer F.Cu) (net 11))
 (segment (start 77.6 4.46) (end 83.46 4.46) (width 1.016) (layer F.Cu) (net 11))
 (segment (start 72.155001 7.385001) (end 72.155001 4.095001) (width 1.016) (layer F.Cu) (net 10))
 (segment (start 72.155001 0.505001) (end 72 0.35) (width 1.016) (layer F.Cu) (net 10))
 (segment (start 72.155001 4.095001) (end 72.155001 0.505001) (width 1.016) (layer F.Cu) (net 10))
 (segment (start 72 0.35) (end 72 -3.4) (width 1.016) (layer F.Cu) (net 10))
 (segment (start 72 -6.64) (end 71.84 -6.8) (width 1.016) (layer F.Cu) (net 10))
 (segment (start 72 -3.4) (end 72 -6.64) (width 1.016) (layer F.Cu) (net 10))
 (segment (start 78.734 -12) (end 81 -12) (width 1.016) (layer F.Cu) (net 10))
 (segment (start 76.928212 -12) (end 78.734 -12) (width 1.016) (layer F.Cu) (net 10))
 (segment (start 71.84 -6.911788) (end 76.928212 -12) (width 1.016) (layer F.Cu) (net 10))
 (segment (start 71.84 -6.8) (end 71.84 -6.911788) (width 1.016) (layer F.Cu) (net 10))
 (segment (start 83.9 11.9) (end 83.6 11.6) (width 1.016) (layer F.Cu) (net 8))
 (segment (start 83.9 18.9) (end 83.9 11.9) (width 1.016) (layer F.Cu) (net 8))
 (segment (start 83.6 11.6) (end 83.6 7.4) (width 1.016) (layer F.Cu) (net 8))
 (segment (start 90.2 7.4) (end 93.8 3.8) (width 1.016) (layer F.Cu) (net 8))
 (segment (start 83.6 7.4) (end 90.2 7.4) (width 1.016) (layer F.Cu) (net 8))
 (segment (start 86.4 -3.6) (end 85.4 -3.6) (width 1.016) (layer F.Cu) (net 8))
 (segment (start 93.8 3.8) (end 86.4 -3.6) (width 1.016) (layer F.Cu) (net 8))
 (segment (start 78.9 18.9) (end 113.9 18.9) (width 1.016) (layer F.Cu) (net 8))
 (segment (start 115.4 15.4) (end 118.9 18.9) (width 1.016) (layer F.Cu) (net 7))
 (segment (start 88.2 -12) (end 100.8 0.6) (width 1.016) (layer F.Cu) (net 7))
 (segment (start 85 -12) (end 88.2 -12) (width 1.016) (layer F.Cu) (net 7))
 (segment (start 100.8 0.6) (end 100.8 11.8) (width 1.016) (layer F.Cu) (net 7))
 (segment (start 100.8 11.8) (end 104.4 15.4) (width 1.016) (layer F.Cu) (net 7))
 (segment (start 104.4 15.4) (end 115.4 15.4) (width 1.016) (layer F.Cu) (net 7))
 (segment (start 68.9 12.1) (end 69.4 11.6) (width 1.016) (layer F.Cu) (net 9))
 (segment (start 68.9 18.9) (end 68.9 12.1) (width 1.016) (layer F.Cu) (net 9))
 (segment (start 43.9 18.9) (end 48.9 18.9) (width 1.016) (layer F.Cu) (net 9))
 (segment (start 48.9 18.9) (end 53.9 18.9) (width 1.016) (layer F.Cu) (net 9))
 (segment (start 53.9 18.9) (end 58.9 18.9) (width 1.016) (layer F.Cu) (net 9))
 (segment (start 58.9 18.9) (end 63.9 18.9) (width 1.016) (layer F.Cu) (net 9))
 (segment (start 63.9 18.9) (end 68.9 18.9) (width 1.016) (layer F.Cu) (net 9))
 (segment (start 68.9 18.9) (end 73.9 18.9) (width 1.016) (layer F.Cu) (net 9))
 (segment (start 69.4 7.43) (end 69.355001 7.385001) (width 1.016) (layer F.Cu) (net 9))
 (segment (start 69.4 11.6) (end 69.4 7.43) (width 1.016) (layer F.Cu) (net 9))
 (segment (start 69.355001 7.385001) (end 69.355001 4.095001) (width 1.016) (layer F.Cu) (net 9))
 (segment (start 69.355001 0.505001) (end 69.2 0.35) (width 1.016) (layer F.Cu) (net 9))
 (segment (start 69.355001 4.095001) (end 69.355001 0.505001) (width 1.016) (layer F.Cu) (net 9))
 (segment (start 69.2 0.35) (end 69.2 -3.4) (width 1.016) (layer F.Cu) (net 9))
 (segment (start 69.2 -6.7) (end 69.3 -6.8) (width 1.016) (layer F.Cu) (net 9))
 (segment (start 69.2 -3.4) (end 69.2 -6.7) (width 1.016) (layer F.Cu) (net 9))
 (segment (start 116.3 -19.2) (end 116.3 -44.2) (width 1.016) (layer F.Cu) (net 3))
 (segment (start 116.3 10.8) (end 116.3 -14.2) (width 1.016) (layer F.Cu) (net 4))
 (segment (start 46.4 -14.2) (end 46.4 10.8) (width 1.016) (layer F.Cu) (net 1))
 (segment (start 46.4 -44.2) (end 46.4 -19.2) (width 1.016) (layer F.Cu) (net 2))
 (segment (start 78.9 -52.3) (end 43.9 -52.3) (width 1.016) (layer F.Cu) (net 5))
 (segment (start 118.9 -52.3) (end 83.9 -52.3) (width 1.016) (layer F.Cu) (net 6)))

